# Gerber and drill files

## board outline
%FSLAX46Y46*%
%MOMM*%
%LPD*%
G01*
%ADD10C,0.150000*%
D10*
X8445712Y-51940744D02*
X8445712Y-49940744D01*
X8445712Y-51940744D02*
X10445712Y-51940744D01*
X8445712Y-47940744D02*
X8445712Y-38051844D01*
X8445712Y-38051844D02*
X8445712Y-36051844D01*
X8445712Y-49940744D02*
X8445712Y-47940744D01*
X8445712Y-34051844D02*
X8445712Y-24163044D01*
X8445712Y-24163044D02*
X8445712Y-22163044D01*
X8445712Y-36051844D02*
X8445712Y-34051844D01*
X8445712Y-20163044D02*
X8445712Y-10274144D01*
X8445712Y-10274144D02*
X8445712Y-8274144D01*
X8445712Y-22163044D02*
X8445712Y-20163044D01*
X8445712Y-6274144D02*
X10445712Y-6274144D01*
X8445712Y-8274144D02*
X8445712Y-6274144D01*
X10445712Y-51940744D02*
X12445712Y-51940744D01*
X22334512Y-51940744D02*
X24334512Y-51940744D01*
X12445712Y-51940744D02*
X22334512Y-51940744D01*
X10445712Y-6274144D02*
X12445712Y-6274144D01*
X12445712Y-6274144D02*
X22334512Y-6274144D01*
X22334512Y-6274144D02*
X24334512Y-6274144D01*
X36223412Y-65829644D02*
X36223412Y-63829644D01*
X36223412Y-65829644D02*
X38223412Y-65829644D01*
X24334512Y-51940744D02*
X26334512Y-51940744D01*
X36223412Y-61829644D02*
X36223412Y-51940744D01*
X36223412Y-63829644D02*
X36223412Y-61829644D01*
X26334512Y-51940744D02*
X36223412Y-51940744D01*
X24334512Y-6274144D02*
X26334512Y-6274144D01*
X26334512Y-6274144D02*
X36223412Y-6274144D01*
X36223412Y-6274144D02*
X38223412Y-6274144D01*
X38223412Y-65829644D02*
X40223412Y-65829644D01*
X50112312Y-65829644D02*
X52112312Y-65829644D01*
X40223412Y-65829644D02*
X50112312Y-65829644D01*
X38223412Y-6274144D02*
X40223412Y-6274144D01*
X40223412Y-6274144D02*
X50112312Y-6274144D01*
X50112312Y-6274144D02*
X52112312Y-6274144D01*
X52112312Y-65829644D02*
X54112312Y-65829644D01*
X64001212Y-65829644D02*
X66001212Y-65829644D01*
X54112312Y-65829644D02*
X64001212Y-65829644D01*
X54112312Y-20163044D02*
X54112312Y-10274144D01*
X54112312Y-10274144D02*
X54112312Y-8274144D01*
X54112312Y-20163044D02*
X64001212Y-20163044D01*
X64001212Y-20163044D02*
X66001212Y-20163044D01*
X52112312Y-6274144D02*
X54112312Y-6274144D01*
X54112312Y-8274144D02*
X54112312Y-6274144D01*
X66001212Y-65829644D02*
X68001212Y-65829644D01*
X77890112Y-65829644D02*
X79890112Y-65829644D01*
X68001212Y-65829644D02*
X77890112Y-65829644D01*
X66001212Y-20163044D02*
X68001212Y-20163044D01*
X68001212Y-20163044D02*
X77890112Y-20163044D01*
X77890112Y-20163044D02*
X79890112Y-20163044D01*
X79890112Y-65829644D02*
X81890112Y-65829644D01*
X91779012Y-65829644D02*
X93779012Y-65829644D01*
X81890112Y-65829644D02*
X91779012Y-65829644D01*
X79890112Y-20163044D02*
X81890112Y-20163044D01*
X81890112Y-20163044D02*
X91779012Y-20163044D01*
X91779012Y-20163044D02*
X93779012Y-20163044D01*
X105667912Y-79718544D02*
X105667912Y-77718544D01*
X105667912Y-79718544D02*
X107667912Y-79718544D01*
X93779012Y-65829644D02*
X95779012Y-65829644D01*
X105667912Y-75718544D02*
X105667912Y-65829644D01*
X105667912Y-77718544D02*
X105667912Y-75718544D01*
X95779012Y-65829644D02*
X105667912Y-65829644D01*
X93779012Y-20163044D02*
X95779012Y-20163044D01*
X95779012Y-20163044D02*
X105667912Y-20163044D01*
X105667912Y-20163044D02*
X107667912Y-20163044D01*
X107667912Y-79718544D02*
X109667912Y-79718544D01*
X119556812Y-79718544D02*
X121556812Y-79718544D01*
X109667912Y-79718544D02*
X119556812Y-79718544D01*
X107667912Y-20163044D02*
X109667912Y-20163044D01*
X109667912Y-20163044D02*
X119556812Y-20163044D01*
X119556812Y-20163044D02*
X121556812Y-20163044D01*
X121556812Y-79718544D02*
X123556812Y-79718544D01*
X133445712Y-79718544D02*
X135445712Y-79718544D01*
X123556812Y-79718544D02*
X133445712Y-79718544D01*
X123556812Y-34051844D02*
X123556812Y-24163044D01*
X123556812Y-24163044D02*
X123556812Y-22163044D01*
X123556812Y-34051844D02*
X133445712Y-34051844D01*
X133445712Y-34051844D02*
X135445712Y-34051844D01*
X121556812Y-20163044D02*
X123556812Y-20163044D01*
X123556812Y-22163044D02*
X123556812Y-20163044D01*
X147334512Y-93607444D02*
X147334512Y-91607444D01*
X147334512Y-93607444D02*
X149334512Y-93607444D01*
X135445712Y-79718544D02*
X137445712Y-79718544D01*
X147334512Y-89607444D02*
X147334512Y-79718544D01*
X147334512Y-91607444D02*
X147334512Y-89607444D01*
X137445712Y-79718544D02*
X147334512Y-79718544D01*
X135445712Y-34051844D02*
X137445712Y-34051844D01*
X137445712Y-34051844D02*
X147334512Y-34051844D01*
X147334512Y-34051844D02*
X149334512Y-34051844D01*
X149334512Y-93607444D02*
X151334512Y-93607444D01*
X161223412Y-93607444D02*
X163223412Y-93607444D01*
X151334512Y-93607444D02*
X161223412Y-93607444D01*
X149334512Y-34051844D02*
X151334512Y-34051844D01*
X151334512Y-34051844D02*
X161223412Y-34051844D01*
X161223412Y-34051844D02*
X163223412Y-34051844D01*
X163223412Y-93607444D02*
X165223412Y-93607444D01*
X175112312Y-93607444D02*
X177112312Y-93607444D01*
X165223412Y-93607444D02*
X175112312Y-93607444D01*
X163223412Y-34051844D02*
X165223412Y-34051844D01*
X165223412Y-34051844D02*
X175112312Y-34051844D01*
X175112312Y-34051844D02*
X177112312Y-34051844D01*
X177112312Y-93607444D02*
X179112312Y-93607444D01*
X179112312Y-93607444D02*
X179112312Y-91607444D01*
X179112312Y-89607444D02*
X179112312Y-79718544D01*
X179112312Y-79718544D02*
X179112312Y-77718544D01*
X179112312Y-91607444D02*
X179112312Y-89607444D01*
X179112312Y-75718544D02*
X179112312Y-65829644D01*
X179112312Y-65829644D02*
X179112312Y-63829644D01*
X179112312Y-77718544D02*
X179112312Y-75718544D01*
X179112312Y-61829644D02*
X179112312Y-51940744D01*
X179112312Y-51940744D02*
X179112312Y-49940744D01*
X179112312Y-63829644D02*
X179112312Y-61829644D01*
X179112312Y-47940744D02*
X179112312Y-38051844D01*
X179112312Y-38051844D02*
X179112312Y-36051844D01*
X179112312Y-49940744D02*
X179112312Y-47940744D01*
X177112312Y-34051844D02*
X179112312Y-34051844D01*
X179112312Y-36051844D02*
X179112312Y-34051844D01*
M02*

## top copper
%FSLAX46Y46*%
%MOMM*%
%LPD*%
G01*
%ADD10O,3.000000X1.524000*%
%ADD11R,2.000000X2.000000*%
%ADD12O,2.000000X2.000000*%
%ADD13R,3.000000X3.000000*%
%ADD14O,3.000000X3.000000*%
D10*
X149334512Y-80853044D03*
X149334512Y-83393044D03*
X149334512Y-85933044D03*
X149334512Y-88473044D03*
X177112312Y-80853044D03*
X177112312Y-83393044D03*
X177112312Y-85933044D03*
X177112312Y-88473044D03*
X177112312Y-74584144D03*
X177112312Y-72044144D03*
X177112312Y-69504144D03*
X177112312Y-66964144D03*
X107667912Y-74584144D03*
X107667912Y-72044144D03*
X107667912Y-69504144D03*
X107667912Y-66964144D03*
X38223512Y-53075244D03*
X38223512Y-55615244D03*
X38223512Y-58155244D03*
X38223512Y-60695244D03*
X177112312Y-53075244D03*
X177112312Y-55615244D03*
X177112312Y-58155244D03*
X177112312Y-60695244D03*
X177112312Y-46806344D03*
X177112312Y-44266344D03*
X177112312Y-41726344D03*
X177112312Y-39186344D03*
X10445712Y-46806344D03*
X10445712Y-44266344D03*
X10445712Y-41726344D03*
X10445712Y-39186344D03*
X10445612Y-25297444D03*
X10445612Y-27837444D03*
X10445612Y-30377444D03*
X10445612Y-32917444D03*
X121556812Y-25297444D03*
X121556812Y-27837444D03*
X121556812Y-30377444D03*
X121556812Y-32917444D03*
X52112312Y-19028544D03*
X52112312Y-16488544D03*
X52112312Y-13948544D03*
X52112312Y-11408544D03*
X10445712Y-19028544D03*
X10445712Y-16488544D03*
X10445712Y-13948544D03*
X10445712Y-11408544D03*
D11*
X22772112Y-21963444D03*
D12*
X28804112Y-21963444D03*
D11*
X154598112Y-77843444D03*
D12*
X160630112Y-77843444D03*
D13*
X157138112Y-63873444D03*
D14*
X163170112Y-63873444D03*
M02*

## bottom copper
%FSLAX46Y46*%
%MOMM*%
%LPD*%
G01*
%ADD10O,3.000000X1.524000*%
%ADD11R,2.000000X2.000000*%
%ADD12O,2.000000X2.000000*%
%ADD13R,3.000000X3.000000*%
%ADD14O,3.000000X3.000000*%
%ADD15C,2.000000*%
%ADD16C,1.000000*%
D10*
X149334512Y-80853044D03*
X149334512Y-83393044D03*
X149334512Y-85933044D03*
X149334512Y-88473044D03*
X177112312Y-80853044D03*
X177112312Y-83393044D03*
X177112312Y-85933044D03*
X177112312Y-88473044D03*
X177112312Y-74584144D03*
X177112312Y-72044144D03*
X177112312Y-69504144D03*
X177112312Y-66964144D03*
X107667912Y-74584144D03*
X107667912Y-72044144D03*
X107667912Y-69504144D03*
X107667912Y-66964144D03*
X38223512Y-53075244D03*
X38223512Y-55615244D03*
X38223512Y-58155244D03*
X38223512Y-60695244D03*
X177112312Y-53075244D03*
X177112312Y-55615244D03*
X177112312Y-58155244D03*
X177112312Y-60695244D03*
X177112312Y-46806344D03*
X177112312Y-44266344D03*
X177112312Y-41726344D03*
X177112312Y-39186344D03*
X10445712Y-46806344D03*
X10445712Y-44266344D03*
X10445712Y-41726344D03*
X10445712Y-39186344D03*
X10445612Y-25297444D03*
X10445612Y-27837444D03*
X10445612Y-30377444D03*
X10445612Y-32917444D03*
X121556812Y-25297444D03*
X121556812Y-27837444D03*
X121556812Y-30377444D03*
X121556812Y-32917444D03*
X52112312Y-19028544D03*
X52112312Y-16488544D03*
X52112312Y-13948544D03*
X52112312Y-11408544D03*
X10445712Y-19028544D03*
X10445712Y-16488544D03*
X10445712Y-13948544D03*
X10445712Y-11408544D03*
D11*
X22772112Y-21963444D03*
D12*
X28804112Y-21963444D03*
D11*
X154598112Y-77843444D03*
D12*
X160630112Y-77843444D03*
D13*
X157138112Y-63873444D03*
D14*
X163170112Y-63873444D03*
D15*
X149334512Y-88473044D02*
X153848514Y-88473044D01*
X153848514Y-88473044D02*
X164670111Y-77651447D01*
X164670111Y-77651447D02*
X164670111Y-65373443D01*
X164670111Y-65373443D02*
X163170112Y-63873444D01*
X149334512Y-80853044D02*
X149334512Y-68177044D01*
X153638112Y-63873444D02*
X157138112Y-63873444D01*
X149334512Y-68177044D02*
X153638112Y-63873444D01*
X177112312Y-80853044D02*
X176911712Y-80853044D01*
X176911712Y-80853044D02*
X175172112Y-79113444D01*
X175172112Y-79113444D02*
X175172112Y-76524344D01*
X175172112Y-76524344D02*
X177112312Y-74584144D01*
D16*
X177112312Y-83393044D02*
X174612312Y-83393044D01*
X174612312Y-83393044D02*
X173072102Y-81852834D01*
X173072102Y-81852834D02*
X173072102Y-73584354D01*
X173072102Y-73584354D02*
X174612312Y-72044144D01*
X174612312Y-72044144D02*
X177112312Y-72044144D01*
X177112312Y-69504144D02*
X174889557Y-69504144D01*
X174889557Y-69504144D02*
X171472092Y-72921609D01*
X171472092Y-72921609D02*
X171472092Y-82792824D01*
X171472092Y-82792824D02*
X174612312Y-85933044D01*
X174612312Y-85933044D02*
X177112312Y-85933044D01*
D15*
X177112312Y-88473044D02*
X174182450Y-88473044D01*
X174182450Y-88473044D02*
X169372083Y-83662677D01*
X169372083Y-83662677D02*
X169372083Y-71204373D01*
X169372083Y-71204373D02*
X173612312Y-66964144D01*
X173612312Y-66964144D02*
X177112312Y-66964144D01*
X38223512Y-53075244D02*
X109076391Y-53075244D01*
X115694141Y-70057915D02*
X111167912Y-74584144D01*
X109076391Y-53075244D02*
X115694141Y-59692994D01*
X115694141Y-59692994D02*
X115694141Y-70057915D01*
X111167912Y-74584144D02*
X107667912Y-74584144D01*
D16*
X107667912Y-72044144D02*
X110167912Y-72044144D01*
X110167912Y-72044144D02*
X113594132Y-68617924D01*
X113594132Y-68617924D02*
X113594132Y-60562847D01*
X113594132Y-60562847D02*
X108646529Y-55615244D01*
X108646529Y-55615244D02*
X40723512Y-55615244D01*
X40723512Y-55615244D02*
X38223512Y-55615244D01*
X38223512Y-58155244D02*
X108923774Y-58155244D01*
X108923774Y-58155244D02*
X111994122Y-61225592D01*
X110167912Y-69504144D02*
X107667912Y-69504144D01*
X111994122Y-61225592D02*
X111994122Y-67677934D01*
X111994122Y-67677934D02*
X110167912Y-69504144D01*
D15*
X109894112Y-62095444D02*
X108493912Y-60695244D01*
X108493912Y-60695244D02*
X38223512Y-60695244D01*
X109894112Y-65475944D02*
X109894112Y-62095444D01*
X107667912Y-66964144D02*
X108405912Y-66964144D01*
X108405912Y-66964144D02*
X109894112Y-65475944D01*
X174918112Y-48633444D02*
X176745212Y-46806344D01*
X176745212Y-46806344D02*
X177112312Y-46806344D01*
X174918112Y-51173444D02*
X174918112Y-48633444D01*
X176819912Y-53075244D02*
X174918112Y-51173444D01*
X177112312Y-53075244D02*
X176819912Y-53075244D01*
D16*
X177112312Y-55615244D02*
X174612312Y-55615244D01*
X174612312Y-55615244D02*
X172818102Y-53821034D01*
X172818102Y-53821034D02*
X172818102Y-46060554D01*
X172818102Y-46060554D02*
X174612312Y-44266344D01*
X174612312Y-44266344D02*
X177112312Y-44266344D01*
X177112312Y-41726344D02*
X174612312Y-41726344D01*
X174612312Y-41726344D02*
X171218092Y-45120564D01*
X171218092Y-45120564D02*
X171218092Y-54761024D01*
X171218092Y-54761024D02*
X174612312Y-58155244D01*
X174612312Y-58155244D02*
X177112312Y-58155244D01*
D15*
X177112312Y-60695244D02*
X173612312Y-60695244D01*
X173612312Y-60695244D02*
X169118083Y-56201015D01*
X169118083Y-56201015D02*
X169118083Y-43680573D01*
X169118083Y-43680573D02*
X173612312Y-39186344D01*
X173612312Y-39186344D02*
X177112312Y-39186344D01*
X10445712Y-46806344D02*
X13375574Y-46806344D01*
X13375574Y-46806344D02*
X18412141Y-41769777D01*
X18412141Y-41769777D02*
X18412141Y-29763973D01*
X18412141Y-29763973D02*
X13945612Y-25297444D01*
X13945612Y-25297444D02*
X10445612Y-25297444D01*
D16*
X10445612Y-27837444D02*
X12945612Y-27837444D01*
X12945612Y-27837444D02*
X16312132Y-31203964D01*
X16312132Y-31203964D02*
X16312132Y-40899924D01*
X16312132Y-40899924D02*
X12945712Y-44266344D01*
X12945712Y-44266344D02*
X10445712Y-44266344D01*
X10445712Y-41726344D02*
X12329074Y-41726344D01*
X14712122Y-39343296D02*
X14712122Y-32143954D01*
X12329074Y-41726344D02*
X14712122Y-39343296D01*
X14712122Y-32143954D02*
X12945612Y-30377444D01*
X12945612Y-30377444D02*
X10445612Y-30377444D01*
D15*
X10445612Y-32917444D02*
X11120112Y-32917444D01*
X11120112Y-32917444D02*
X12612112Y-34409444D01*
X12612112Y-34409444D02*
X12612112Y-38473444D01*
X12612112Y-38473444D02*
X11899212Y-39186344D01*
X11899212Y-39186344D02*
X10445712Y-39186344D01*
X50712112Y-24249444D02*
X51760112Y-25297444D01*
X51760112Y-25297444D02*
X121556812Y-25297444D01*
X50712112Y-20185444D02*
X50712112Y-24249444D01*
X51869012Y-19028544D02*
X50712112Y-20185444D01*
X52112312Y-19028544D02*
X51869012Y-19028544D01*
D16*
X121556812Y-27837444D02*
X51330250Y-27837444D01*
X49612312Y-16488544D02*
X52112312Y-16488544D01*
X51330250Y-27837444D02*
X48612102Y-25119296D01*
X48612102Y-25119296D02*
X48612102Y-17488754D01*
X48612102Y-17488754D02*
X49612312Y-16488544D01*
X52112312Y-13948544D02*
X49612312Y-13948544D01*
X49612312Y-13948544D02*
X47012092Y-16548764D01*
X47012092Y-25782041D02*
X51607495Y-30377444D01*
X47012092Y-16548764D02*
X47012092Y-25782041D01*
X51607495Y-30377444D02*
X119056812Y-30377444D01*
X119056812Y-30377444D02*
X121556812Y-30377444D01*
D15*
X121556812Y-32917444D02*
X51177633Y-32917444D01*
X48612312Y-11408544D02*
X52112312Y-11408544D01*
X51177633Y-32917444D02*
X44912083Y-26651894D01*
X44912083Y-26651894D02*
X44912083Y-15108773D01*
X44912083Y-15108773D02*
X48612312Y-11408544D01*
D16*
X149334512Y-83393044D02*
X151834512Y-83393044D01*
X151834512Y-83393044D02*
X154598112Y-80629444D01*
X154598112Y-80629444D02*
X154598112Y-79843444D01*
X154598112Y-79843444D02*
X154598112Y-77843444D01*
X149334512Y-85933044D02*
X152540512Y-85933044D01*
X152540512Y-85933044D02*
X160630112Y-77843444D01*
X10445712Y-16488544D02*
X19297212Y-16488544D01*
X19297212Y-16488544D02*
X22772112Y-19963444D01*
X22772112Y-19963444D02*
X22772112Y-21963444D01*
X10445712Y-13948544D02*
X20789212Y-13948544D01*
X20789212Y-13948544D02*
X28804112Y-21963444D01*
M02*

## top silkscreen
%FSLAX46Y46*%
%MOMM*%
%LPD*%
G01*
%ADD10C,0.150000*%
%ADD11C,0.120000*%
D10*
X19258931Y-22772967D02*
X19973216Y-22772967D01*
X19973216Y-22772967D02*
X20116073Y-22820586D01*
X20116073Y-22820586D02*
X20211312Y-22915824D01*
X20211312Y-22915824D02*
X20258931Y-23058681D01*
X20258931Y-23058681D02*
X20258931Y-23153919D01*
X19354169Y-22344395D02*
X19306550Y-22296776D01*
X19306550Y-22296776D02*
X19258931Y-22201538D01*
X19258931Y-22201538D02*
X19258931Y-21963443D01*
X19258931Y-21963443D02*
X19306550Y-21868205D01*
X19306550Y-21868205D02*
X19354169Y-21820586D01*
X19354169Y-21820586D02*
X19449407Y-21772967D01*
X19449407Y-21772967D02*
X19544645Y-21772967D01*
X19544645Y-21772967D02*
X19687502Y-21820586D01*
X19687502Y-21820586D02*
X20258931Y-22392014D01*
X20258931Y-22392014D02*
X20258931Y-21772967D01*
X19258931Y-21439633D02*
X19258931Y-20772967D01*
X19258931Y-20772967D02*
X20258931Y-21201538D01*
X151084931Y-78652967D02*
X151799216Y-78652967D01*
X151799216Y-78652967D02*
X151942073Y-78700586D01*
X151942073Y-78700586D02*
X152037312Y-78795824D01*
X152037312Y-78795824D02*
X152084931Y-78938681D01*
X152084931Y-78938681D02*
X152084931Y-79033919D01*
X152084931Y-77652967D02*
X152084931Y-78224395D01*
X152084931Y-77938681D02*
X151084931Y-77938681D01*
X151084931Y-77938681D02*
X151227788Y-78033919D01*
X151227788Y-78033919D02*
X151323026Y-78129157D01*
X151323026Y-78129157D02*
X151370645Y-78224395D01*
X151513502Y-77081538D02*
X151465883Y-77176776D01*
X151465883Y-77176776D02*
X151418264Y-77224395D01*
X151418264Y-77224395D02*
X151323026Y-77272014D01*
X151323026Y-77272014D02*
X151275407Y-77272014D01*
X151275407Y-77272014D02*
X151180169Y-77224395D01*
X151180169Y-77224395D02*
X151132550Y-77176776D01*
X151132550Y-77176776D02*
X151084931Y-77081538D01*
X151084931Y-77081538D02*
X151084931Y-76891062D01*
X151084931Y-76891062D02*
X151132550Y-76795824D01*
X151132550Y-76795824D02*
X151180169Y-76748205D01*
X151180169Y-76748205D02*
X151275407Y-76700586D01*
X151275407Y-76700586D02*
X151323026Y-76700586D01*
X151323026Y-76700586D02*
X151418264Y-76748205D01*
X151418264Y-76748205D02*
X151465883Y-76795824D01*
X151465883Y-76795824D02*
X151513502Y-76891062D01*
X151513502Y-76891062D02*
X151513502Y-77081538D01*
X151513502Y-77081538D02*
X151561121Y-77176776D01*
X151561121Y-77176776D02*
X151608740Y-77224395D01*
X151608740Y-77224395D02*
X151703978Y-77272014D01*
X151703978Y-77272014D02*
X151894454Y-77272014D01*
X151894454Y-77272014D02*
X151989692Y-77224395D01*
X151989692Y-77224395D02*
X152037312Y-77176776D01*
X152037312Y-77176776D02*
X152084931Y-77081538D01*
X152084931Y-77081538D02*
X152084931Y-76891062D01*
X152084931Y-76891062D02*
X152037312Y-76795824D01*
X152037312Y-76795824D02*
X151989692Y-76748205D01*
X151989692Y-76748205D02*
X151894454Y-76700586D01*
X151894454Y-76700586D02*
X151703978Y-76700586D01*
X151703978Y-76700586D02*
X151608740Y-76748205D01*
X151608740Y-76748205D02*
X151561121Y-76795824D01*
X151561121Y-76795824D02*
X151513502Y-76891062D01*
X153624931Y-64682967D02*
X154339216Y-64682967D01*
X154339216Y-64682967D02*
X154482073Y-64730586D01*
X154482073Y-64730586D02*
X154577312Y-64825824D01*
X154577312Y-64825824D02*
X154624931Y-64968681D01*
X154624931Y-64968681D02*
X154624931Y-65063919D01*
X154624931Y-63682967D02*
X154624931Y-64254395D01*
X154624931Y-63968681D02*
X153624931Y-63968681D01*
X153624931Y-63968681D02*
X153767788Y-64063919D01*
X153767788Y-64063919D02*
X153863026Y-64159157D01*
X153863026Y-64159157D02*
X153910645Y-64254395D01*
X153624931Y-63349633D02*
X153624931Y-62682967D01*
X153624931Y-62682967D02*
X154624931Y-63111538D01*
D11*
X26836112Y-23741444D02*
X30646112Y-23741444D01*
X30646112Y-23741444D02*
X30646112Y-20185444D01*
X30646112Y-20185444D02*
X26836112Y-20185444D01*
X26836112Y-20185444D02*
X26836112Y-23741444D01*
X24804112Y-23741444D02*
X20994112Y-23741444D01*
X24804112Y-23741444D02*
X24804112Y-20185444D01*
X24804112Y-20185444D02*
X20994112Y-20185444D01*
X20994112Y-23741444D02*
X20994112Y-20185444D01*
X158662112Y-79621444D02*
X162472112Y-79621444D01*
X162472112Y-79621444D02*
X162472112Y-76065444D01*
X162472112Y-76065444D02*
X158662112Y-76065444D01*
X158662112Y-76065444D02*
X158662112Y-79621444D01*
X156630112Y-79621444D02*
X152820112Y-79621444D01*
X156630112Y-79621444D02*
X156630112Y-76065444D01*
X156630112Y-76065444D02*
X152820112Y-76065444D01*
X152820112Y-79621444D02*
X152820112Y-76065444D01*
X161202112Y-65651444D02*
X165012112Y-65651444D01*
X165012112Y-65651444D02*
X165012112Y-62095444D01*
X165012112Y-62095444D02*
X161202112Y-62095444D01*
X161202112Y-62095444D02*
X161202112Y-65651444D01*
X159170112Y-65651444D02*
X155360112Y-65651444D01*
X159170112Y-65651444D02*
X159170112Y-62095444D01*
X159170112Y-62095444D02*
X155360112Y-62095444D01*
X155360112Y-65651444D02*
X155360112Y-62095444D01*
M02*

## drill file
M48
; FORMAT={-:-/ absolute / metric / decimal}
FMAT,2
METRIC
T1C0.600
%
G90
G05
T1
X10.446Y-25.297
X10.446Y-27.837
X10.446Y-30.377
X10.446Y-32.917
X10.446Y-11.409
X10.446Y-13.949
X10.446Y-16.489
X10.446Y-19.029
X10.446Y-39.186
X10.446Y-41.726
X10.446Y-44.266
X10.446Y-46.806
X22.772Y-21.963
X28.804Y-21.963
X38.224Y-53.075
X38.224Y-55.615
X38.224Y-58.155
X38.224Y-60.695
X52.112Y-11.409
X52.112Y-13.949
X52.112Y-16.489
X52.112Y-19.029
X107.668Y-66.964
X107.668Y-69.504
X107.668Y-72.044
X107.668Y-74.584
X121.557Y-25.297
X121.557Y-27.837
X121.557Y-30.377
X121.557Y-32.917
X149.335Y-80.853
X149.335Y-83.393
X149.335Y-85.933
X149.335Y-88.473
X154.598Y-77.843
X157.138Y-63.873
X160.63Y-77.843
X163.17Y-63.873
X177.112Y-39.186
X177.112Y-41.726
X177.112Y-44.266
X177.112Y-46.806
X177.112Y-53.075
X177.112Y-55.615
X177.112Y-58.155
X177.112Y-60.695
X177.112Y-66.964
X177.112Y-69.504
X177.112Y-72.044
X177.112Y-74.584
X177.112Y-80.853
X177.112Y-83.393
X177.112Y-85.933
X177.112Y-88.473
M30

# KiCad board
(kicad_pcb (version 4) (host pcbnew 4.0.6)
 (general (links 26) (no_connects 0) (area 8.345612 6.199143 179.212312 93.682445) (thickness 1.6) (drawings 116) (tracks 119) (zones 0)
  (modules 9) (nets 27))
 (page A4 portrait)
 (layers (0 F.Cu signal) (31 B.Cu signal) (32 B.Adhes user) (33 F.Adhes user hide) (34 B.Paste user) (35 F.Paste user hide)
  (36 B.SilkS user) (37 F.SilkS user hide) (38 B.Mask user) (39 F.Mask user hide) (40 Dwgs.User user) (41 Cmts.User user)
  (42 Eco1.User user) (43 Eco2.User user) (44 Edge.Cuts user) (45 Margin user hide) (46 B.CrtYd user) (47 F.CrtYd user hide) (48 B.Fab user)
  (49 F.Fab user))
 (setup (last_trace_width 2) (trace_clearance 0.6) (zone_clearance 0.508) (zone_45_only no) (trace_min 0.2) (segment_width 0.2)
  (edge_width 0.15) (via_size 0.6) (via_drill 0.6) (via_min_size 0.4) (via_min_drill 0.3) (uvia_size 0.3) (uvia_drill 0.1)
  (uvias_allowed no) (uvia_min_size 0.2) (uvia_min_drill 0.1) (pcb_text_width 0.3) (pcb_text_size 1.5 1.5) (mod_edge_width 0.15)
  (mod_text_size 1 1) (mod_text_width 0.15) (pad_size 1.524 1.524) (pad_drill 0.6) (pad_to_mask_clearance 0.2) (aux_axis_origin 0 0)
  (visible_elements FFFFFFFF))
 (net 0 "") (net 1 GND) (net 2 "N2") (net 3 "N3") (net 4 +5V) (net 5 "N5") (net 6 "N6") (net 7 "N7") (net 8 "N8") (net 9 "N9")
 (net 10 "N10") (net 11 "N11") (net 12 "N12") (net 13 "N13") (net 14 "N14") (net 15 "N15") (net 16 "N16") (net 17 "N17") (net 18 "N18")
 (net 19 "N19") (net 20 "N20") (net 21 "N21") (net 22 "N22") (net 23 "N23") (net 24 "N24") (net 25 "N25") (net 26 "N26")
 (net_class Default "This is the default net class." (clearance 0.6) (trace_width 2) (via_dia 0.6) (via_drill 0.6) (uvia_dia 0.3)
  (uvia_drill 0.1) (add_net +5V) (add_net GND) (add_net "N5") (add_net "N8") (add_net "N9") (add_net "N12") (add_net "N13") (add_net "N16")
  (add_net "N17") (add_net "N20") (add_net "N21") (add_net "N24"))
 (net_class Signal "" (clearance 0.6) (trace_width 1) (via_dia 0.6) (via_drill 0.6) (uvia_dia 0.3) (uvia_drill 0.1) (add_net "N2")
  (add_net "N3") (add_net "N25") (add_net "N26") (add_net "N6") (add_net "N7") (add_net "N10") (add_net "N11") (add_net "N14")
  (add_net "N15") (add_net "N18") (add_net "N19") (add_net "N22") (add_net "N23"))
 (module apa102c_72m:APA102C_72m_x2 (layer B.Cu) (at 163.223412 84.663044)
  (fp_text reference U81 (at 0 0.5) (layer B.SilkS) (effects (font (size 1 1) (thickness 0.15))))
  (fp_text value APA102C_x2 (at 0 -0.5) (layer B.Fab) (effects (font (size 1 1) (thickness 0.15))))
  (pad 1 thru_hole oval (at -13.8889 -3.81) (size 3 1.524) (drill 0.6) (layers *.Cu *.Mask) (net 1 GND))
  (pad 2 thru_hole oval (at -13.8889 -1.27) (size 3 1.524) (drill 0.6) (layers *.Cu *.Mask) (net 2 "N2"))
  (pad 3 thru_hole oval (at -13.8889 1.27) (size 3 1.524) (drill 0.6) (layers *.Cu *.Mask) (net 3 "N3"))
  (pad 4 thru_hole oval (at -13.8889 3.81) (size 3 1.524) (drill 0.6) (layers *.Cu *.Mask) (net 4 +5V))
  (pad 5 thru_hole oval (at 13.8889 -3.81) (size 3 1.524) (drill 0.6) (layers *.Cu *.Mask) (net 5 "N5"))
  (pad 6 thru_hole oval (at 13.8889 -1.27) (size 3 1.524) (drill 0.6) (layers *.Cu *.Mask) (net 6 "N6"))
  (pad 7 thru_hole oval (at 13.8889 1.27) (size 3 1.524) (drill 0.6) (layers *.Cu *.Mask) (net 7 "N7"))
  (pad 8 thru_hole oval (at 13.8889 3.81) (size 3 1.524) (drill 0.6) (layers *.Cu *.Mask) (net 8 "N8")))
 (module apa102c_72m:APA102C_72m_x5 (layer B.Cu) (at 142.390112 70.774144 180)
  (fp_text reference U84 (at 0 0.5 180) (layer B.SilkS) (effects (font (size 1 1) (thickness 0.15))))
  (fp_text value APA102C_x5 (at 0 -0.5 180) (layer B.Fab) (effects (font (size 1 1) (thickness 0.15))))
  (pad 1 thru_hole oval (at -34.7222 -3.81 180) (size 3 1.524) (drill 0.6) (layers *.Cu *.Mask) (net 5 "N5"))
  (pad 2 thru_hole oval (at -34.7222 -1.27 180) (size 3 1.524) (drill 0.6) (layers *.Cu *.Mask) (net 6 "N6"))
  (pad 3 thru_hole oval (at -34.7222 1.27 180) (size 3 1.524) (drill 0.6) (layers *.Cu *.Mask) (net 7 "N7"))
  (pad 4 thru_hole oval (at -34.7222 3.81 180) (size 3 1.524) (drill 0.6) (layers *.Cu *.Mask) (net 8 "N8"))
  (pad 5 thru_hole oval (at 34.7222 -3.81 180) (size 3 1.524) (drill 0.6) (layers *.Cu *.Mask) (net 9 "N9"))
  (pad 6 thru_hole oval (at 34.7222 -1.27 180) (size 3 1.524) (drill 0.6) (layers *.Cu *.Mask) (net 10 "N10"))
  (pad 7 thru_hole oval (at 34.7222 1.27 180) (size 3 1.524) (drill 0.6) (layers *.Cu *.Mask) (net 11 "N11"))
  (pad 8 thru_hole oval (at 34.7222 3.81 180) (size 3 1.524) (drill 0.6) (layers *.Cu *.Mask) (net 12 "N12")))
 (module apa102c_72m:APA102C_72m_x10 (layer B.Cu) (at 107.667912 56.885244)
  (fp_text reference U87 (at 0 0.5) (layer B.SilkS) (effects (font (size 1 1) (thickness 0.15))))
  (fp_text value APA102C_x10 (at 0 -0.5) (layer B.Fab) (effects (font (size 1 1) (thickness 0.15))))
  (pad 1 thru_hole oval (at -69.4444 -3.81) (size 3 1.524) (drill 0.6) (layers *.Cu *.Mask) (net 9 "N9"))
  (pad 2 thru_hole oval (at -69.4444 -1.27) (size 3 1.524) (drill 0.6) (layers *.Cu *.Mask) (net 10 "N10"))
  (pad 3 thru_hole oval (at -69.4444 1.27) (size 3 1.524) (drill 0.6) (layers *.Cu *.Mask) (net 11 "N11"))
  (pad 4 thru_hole oval (at -69.4444 3.81) (size 3 1.524) (drill 0.6) (layers *.Cu *.Mask) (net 12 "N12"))
  (pad 5 thru_hole oval (at 69.4444 -3.81) (size 3 1.524) (drill 0.6) (layers *.Cu *.Mask) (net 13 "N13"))
  (pad 6 thru_hole oval (at 69.4444 -1.27) (size 3 1.524) (drill 0.6) (layers *.Cu *.Mask) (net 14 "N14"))
  (pad 7 thru_hole oval (at 69.4444 1.27) (size 3 1.524) (drill 0.6) (layers *.Cu *.Mask) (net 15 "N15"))
  (pad 8 thru_hole oval (at 69.4444 3.81) (size 3 1.524) (drill 0.6) (layers *.Cu *.Mask) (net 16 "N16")))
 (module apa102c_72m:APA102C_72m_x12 (layer B.Cu) (at 93.779012 42.996344 180)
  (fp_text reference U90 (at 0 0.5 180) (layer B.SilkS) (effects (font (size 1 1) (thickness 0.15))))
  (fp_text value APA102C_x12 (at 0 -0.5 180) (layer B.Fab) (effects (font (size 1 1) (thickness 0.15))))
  (pad 1 thru_hole oval (at -83.3333 -3.81 180) (size 3 1.524) (drill 0.6) (layers *.Cu *.Mask) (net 13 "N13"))
  (pad 2 thru_hole oval (at -83.3333 -1.27 180) (size 3 1.524) (drill 0.6) (layers *.Cu *.Mask) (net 14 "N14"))
  (pad 3 thru_hole oval (at -83.3333 1.27 180) (size 3 1.524) (drill 0.6) (layers *.Cu *.Mask) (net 15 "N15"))
  (pad 4 thru_hole oval (at -83.3333 3.81 180) (size 3 1.524) (drill 0.6) (layers *.Cu *.Mask) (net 16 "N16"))
  (pad 5 thru_hole oval (at 83.3333 -3.81 180) (size 3 1.524) (drill 0.6) (layers *.Cu *.Mask) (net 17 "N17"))
  (pad 6 thru_hole oval (at 83.3333 -1.27 180) (size 3 1.524) (drill 0.6) (layers *.Cu *.Mask) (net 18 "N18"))
  (pad 7 thru_hole oval (at 83.3333 1.27 180) (size 3 1.524) (drill 0.6) (layers *.Cu *.Mask) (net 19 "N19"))
  (pad 8 thru_hole oval (at 83.3333 3.81 180) (size 3 1.524) (drill 0.6) (layers *.Cu *.Mask) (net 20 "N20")))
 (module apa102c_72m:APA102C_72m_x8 (layer B.Cu) (at 66.001212 29.107444)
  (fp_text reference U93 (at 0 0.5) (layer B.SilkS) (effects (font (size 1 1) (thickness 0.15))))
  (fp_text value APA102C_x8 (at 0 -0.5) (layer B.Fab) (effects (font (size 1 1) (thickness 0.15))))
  (pad 1 thru_hole oval (at -55.5556 -3.81) (size 3 1.524) (drill 0.6) (layers *.Cu *.Mask) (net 17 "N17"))
  (pad 2 thru_hole oval (at -55.5556 -1.27) (size 3 1.524) (drill 0.6) (layers *.Cu *.Mask) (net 18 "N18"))
  (pad 3 thru_hole oval (at -55.5556 1.27) (size 3 1.524) (drill 0.6) (layers *.Cu *.Mask) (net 19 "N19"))
  (pad 4 thru_hole oval (at -55.5556 3.81) (size 3 1.524) (drill 0.6) (layers *.Cu *.Mask) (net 20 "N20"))
  (pad 5 thru_hole oval (at 55.5556 -3.81) (size 3 1.524) (drill 0.6) (layers *.Cu *.Mask) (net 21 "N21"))
  (pad 6 thru_hole oval (at 55.5556 -1.27) (size 3 1.524) (drill 0.6) (layers *.Cu *.Mask) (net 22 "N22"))
  (pad 7 thru_hole oval (at 55.5556 1.27) (size 3 1.524) (drill 0.6) (layers *.Cu *.Mask) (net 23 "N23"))
  (pad 8 thru_hole oval (at 55.5556 3.81) (size 3 1.524) (drill 0.6) (layers *.Cu *.Mask) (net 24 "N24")))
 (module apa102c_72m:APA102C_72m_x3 (layer B.Cu) (at 31.279012 15.218544 180)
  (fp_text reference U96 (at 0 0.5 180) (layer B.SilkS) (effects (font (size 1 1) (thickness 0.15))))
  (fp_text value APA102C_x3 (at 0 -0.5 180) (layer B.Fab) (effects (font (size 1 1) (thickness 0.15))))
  (pad 1 thru_hole oval (at -20.8333 -3.81 180) (size 3 1.524) (drill 0.6) (layers *.Cu *.Mask) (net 21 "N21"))
  (pad 2 thru_hole oval (at -20.8333 -1.27 180) (size 3 1.524) (drill 0.6) (layers *.Cu *.Mask) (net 22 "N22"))
  (pad 3 thru_hole oval (at -20.8333 1.27 180) (size 3 1.524) (drill 0.6) (layers *.Cu *.Mask) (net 23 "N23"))
  (pad 4 thru_hole oval (at -20.8333 3.81 180) (size 3 1.524) (drill 0.6) (layers *.Cu *.Mask) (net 24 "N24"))
  (pad 5 thru_hole oval (at 20.8333 -3.81 180) (size 3 1.524) (drill 0.6) (layers *.Cu *.Mask))
  (pad 6 thru_hole oval (at 20.8333 -1.27 180) (size 3 1.524) (drill 0.6) (layers *.Cu *.Mask) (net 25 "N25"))
  (pad 7 thru_hole oval (at 20.8333 1.27 180) (size 3 1.524) (drill 0.6) (layers *.Cu *.Mask) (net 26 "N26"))
  (pad 8 thru_hole oval (at 20.8333 3.81 180) (size 3 1.524) (drill 0.6) (layers *.Cu *.Mask)))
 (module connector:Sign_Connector (layer F.Cu) (at 24.804112 21.963444 90)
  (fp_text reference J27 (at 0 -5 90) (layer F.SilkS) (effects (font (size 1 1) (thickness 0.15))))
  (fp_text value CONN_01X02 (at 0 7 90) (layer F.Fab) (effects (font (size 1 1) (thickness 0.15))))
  (fp_line (start -1.778 2.032) (end -1.778 5.842) (layer F.SilkS) (width 0.12))
  (fp_line (start -1.778 5.842) (end 1.778 5.842) (layer F.SilkS) (width 0.12))
  (fp_line (start 1.778 5.842) (end 1.778 2.032) (layer F.SilkS) (width 0.12))
  (fp_line (start 1.778 2.032) (end -1.778 2.032) (layer F.SilkS) (width 0.12))
  (fp_line (start -1.778 0) (end -1.778 -3.81) (layer F.SilkS) (width 0.12))
  (fp_line (start -1.778 0) (end 1.778 0) (layer F.SilkS) (width 0.12))
  (fp_line (start 1.778 0) (end 1.778 -3.81) (layer F.SilkS) (width 0.12))
  (fp_line (start -1.778 -3.81) (end 1.778 -3.81) (layer F.SilkS) (width 0.12))
  (pad 1 thru_hole rect (at 0 -2.032 90) (size 2 2) (drill 0.6) (layers *.Cu *.Mask) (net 25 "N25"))
  (pad 2 thru_hole oval (at 0 4 90) (size 2 2) (drill 0.6) (layers *.Cu *.Mask) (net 26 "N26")))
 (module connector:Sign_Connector (layer F.Cu) (at 156.630112 77.843444 90)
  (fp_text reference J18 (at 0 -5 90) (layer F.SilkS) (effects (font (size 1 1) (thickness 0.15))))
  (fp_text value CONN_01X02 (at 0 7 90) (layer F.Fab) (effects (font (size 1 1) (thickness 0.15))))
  (fp_line (start -1.778 2.032) (end -1.778 5.842) (layer F.SilkS) (width 0.12))
  (fp_line (start -1.778 5.842) (end 1.778 5.842) (layer F.SilkS) (width 0.12))
  (fp_line (start 1.778 5.842) (end 1.778 2.032) (layer F.SilkS) (width 0.12))
  (fp_line (start 1.778 2.032) (end -1.778 2.032) (layer F.SilkS) (width 0.12))
  (fp_line (start -1.778 0) (end -1.778 -3.81) (layer F.SilkS) (width 0.12))
  (fp_line (start -1.778 0) (end 1.778 0) (layer F.SilkS) (width 0.12))
  (fp_line (start 1.778 0) (end 1.778 -3.81) (layer F.SilkS) (width 0.12))
  (fp_line (start -1.778 -3.81) (end 1.778 -3.81) (layer F.SilkS) (width 0.12))
  (pad 1 thru_hole rect (at 0 -2.032 90) (size 2 2) (drill 0.6) (layers *.Cu *.Mask) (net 2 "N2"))
  (pad 2 thru_hole oval (at 0 4 90) (size 2 2) (drill 0.6) (layers *.Cu *.Mask) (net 3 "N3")))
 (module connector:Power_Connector (layer F.Cu) (at 159.170112 63.873444 90)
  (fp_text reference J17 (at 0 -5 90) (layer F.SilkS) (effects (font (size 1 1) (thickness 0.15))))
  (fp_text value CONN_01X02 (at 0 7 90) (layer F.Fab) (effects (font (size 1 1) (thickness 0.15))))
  (fp_line (start -1.778 2.032) (end -1.778 5.842) (layer F.SilkS) (width 0.12))
  (fp_line (start -1.778 5.842) (end 1.778 5.842) (layer F.SilkS) (width 0.12))
  (fp_line (start 1.778 5.842) (end 1.778 2.032) (layer F.SilkS) (width 0.12))
  (fp_line (start 1.778 2.032) (end -1.778 2.032) (layer F.SilkS) (width 0.12))
  (fp_line (start -1.778 0) (end -1.778 -3.81) (layer F.SilkS) (width 0.12))
  (fp_line (start -1.778 0) (end 1.778 0) (layer F.SilkS) (width 0.12))
  (fp_line (start 1.778 0) (end 1.778 -3.81) (layer F.SilkS) (width 0.12))
  (fp_line (start -1.778 -3.81) (end 1.778 -3.81) (layer F.SilkS) (width 0.12))
  (pad 1 thru_hole rect (at 0 -2.032 90) (size 3 3) (drill 0.6) (layers *.Cu *.Mask) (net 1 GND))
  (pad 2 thru_hole oval (at 0 4 90) (size 3 3) (drill 0.6) (layers *.Cu *.Mask) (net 4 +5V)))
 (gr_line (start 8.445712 51.940744) (end 8.445712 49.940744) (layer Edge.Cuts) (width 0.15))
 (gr_line (start 8.445712 51.940744) (end 10.445712 51.940744) (layer Edge.Cuts) (width 0.15))
 (gr_line (start 8.445712 47.940744) (end 8.445712 38.051844) (layer Edge.Cuts) (width 0.15))
 (gr_line (start 8.445712 38.051844) (end 8.445712 36.051844) (layer Edge.Cuts) (width 0.15))
 (gr_line (start 8.445712 49.940744) (end 8.445712 47.940744) (layer Edge.Cuts) (width 0.15))
 (gr_line (start 8.445712 34.051844) (end 8.445712 24.163044) (layer Edge.Cuts) (width 0.15))
 (gr_line (start 8.445712 24.163044) (end 8.445712 22.163044) (layer Edge.Cuts) (width 0.15))
 (gr_line (start 8.445712 36.051844) (end 8.445712 34.051844) (layer Edge.Cuts) (width 0.15))
 (gr_line (start 8.445712 20.163044) (end 8.445712 10.274144) (layer Edge.Cuts) (width 0.15))
 (gr_line (start 8.445712 10.274144) (end 8.445712 8.274144) (layer Edge.Cuts) (width 0.15))
 (gr_line (start 8.445712 22.163044) (end 8.445712 20.163044) (layer Edge.Cuts) (width 0.15))
 (gr_line (start 8.445712 6.274144) (end 10.445712 6.274144) (layer Edge.Cuts) (width 0.15))
 (gr_line (start 8.445712 8.274144) (end 8.445712 6.274144) (layer Edge.Cuts) (width 0.15))
 (gr_line (start 10.445712 51.940744) (end 12.445712 51.940744) (layer Edge.Cuts) (width 0.15))
 (gr_line (start 22.334512 51.940744) (end 24.334512 51.940744) (layer Edge.Cuts) (width 0.15))
 (gr_line (start 12.445712 51.940744) (end 22.334512 51.940744) (layer Edge.Cuts) (width 0.15))
 (gr_line (start 10.445712 6.274144) (end 12.445712 6.274144) (layer Edge.Cuts) (width 0.15))
 (gr_line (start 12.445712 6.274144) (end 22.334512 6.274144) (layer Edge.Cuts) (width 0.15))
 (gr_line (start 22.334512 6.274144) (end 24.334512 6.274144) (layer Edge.Cuts) (width 0.15))
 (gr_line (start 36.223412 65.829644) (end 36.223412 63.829644) (layer Edge.Cuts) (width 0.15))
 (gr_line (start 36.223412 65.829644) (end 38.223412 65.829644) (layer Edge.Cuts) (width 0.15))
 (gr_line (start 24.334512 51.940744) (end 26.334512 51.940744) (layer Edge.Cuts) (width 0.15))
 (gr_line (start 36.223412 61.829644) (end 36.223412 51.940744) (layer Edge.Cuts) (width 0.15))
 (gr_line (start 36.223412 63.829644) (end 36.223412 61.829644) (layer Edge.Cuts) (width 0.15))
 (gr_line (start 26.334512 51.940744) (end 36.223412 51.940744) (layer Edge.Cuts) (width 0.15))
 (gr_line (start 24.334512 6.274144) (end 26.334512 6.274144) (layer Edge.Cuts) (width 0.15))
 (gr_line (start 26.334512 6.274144) (end 36.223412 6.274144) (layer Edge.Cuts) (width 0.15))
 (gr_line (start 36.223412 6.274144) (end 38.223412 6.274144) (layer Edge.Cuts) (width 0.15))
 (gr_line (start 38.223412 65.829644) (end 40.223412 65.829644) (layer Edge.Cuts) (width 0.15))
 (gr_line (start 50.112312 65.829644) (end 52.112312 65.829644) (layer Edge.Cuts) (width 0.15))
 (gr_line (start 40.223412 65.829644) (end 50.112312 65.829644) (layer Edge.Cuts) (width 0.15))
 (gr_line (start 38.223412 6.274144) (end 40.223412 6.274144) (layer Edge.Cuts) (width 0.15))
 (gr_line (start 40.223412 6.274144) (end 50.112312 6.274144) (layer Edge.Cuts) (width 0.15))
 (gr_line (start 50.112312 6.274144) (end 52.112312 6.274144) (layer Edge.Cuts) (width 0.15))
 (gr_line (start 52.112312 65.829644) (end 54.112312 65.829644) (layer Edge.Cuts) (width 0.15))
 (gr_line (start 64.001212 65.829644) (end 66.001212 65.829644) (layer Edge.Cuts) (width 0.15))
 (gr_line (start 54.112312 65.829644) (end 64.001212 65.829644) (layer Edge.Cuts) (width 0.15))
 (gr_line (start 54.112312 20.163044) (end 54.112312 10.274144) (layer Edge.Cuts) (width 0.15))
 (gr_line (start 54.112312 10.274144) (end 54.112312 8.274144) (layer Edge.Cuts) (width 0.15))
 (gr_line (start 54.112312 20.163044) (end 64.001212 20.163044) (layer Edge.Cuts) (width 0.15))
 (gr_line (start 64.001212 20.163044) (end 66.001212 20.163044) (layer Edge.Cuts) (width 0.15))
 (gr_line (start 52.112312 6.274144) (end 54.112312 6.274144) (layer Edge.Cuts) (width 0.15))
 (gr_line (start 54.112312 8.274144) (end 54.112312 6.274144) (layer Edge.Cuts) (width 0.15))
 (gr_line (start 66.001212 65.829644) (end 68.001212 65.829644) (layer Edge.Cuts) (width 0.15))
 (gr_line (start 77.890112 65.829644) (end 79.890112 65.829644) (layer Edge.Cuts) (width 0.15))
 (gr_line (start 68.001212 65.829644) (end 77.890112 65.829644) (layer Edge.Cuts) (width 0.15))
 (gr_line (start 66.001212 20.163044) (end 68.001212 20.163044) (layer Edge.Cuts) (width 0.15))
 (gr_line (start 68.001212 20.163044) (end 77.890112 20.163044) (layer Edge.Cuts) (width 0.15))
 (gr_line (start 77.890112 20.163044) (end 79.890112 20.163044) (layer Edge.Cuts) (width 0.15))
 (gr_line (start 79.890112 65.829644) (end 81.890112 65.829644) (layer Edge.Cuts) (width 0.15))
 (gr_line (start 91.779012 65.829644) (end 93.779012 65.829644) (layer Edge.Cuts) (width 0.15))
 (gr_line (start 81.890112 65.829644) (end 91.779012 65.829644) (layer Edge.Cuts) (width 0.15))
 (gr_line (start 79.890112 20.163044) (end 81.890112 20.163044) (layer Edge.Cuts) (width 0.15))
 (gr_line (start 81.890112 20.163044) (end 91.779012 20.163044) (layer Edge.Cuts) (width 0.15))
 (gr_line (start 91.779012 20.163044) (end 93.779012 20.163044) (layer Edge.Cuts) (width 0.15))
 (gr_line (start 105.667912 79.718544) (end 105.667912 77.718544) (layer Edge.Cuts) (width 0.15))
 (gr_line (start 105.667912 79.718544) (end 107.667912 79.718544) (layer Edge.Cuts) (width 0.15))
 (gr_line (start 93.779012 65.829644) (end 95.779012 65.829644) (layer Edge.Cuts) (width 0.15))
 (gr_line (start 105.667912 75.718544) (end 105.667912 65.829644) (layer Edge.Cuts) (width 0.15))
 (gr_line (start 105.667912 77.718544) (end 105.667912 75.718544) (layer Edge.Cuts) (width 0.15))
 (gr_line (start 95.779012 65.829644) (end 105.667912 65.829644) (layer Edge.Cuts) (width 0.15))
 (gr_line (start 93.779012 20.163044) (end 95.779012 20.163044) (layer Edge.Cuts) (width 0.15))
 (gr_line (start 95.779012 20.163044) (end 105.667912 20.163044) (layer Edge.Cuts) (width 0.15))
 (gr_line (start 105.667912 20.163044) (end 107.667912 20.163044) (layer Edge.Cuts) (width 0.15))
 (gr_line (start 107.667912 79.718544) (end 109.667912 79.718544) (layer Edge.Cuts) (width 0.15))
 (gr_line (start 119.556812 79.718544) (end 121.556812 79.718544) (layer Edge.Cuts) (width 0.15))
 (gr_line (start 109.667912 79.718544) (end 119.556812 79.718544) (layer Edge.Cuts) (width 0.15))
 (gr_line (start 107.667912 20.163044) (end 109.667912 20.163044) (layer Edge.Cuts) (width 0.15))
 (gr_line (start 109.667912 20.163044) (end 119.556812 20.163044) (layer Edge.Cuts) (width 0.15))
 (gr_line (start 119.556812 20.163044) (end 121.556812 20.163044) (layer Edge.Cuts) (width 0.15))
 (gr_line (start 121.556812 79.718544) (end 123.556812 79.718544) (layer Edge.Cuts) (width 0.15))
 (gr_line (start 133.445712 79.718544) (end 135.445712 79.718544) (layer Edge.Cuts) (width 0.15))
 (gr_line (start 123.556812 79.718544) (end 133.445712 79.718544) (layer Edge.Cuts) (width 0.15))
 (gr_line (start 123.556812 34.051844) (end 123.556812 24.163044) (layer Edge.Cuts) (width 0.15))
 (gr_line (start 123.556812 24.163044) (end 123.556812 22.163044) (layer Edge.Cuts) (width 0.15))
 (gr_line (start 123.556812 34.051844) (end 133.445712 34.051844) (layer Edge.Cuts) (width 0.15))
 (gr_line (start 133.445712 34.051844) (end 135.445712 34.051844) (layer Edge.Cuts) (width 0.15))
 (gr_line (start 121.556812 20.163044) (end 123.556812 20.163044) (layer Edge.Cuts) (width 0.15))
 (gr_line (start 123.556812 22.163044) (end 123.556812 20.163044) (layer Edge.Cuts) (width 0.15))
 (gr_line (start 147.334512 93.607444) (end 147.334512 91.607444) (layer Edge.Cuts) (width 0.15))
 (gr_line (start 147.334512 93.607444) (end 149.334512 93.607444) (layer Edge.Cuts) (width 0.15))
 (gr_line (start 135.445712 79.718544) (end 137.445712 79.718544) (layer Edge.Cuts) (width 0.15))
 (gr_line (start 147.334512 89.607444) (end 147.334512 79.718544) (layer Edge.Cuts) (width 0.15))
 (gr_line (start 147.334512 91.607444) (end 147.334512 89.607444) (layer Edge.Cuts) (width 0.15))
 (gr_line (start 137.445712 79.718544) (end 147.334512 79.718544) (layer Edge.Cuts) (width 0.15))
 (gr_line (start 135.445712 34.051844) (end 137.445712 34.051844) (layer Edge.Cuts) (width 0.15))
 (gr_line (start 137.445712 34.051844) (end 147.334512 34.051844) (layer Edge.Cuts) (width 0.15))
 (gr_line (start 147.334512 34.051844) (end 149.334512 34.051844) (layer Edge.Cuts) (width 0.15))
 (gr_line (start 149.334512 93.607444) (end 151.334512 93.607444) (layer Edge.Cuts) (width 0.15))
 (gr_line (start 161.223412 93.607444) (end 163.223412 93.607444) (layer Edge.Cuts) (width 0.15))
 (gr_line (start 151.334512 93.607444) (end 161.223412 93.607444) (layer Edge.Cuts) (width 0.15))
 (gr_line (start 149.334512 34.051844) (end 151.334512 34.051844) (layer Edge.Cuts) (width 0.15))
 (gr_line (start 151.334512 34.051844) (end 161.223412 34.051844) (layer Edge.Cuts) (width 0.15))
 (gr_line (start 161.223412 34.051844) (end 163.223412 34.051844) (layer Edge.Cuts) (width 0.15))
 (gr_line (start 163.223412 93.607444) (end 165.223412 93.607444) (layer Edge.Cuts) (width 0.15))
 (gr_line (start 175.112312 93.607444) (end 177.112312 93.607444) (layer Edge.Cuts) (width 0.15))
 (gr_line (start 165.223412 93.607444) (end 175.112312 93.607444) (layer Edge.Cuts) (width 0.15))
 (gr_line (start 163.223412 34.051844) (end 165.223412 34.051844) (layer Edge.Cuts) (width 0.15))
 (gr_line (start 165.223412 34.051844) (end 175.112312 34.051844) (layer Edge.Cuts) (width 0.15))
 (gr_line (start 175.112312 34.051844) (end 177.112312 34.051844) (layer Edge.Cuts) (width 0.15))
 (gr_line (start 177.112312 93.607444) (end 179.112312 93.607444) (layer Edge.Cuts) (width 0.15))
 (gr_line (start 179.112312 93.607444) (end 179.112312 91.607444) (layer Edge.Cuts) (width 0.15))
 (gr_line (start 179.112312 89.607444) (end 179.112312 79.718544) (layer Edge.Cuts) (width 0.15))
 (gr_line (start 179.112312 79.718544) (end 179.112312 77.718544) (layer Edge.Cuts) (width 0.15))
 (gr_line (start 179.112312 91.607444) (end 179.112312 89.607444) (layer Edge.Cuts) (width 0.15))
 (gr_line (start 179.112312 75.718544) (end 179.112312 65.829644) (layer Edge.Cuts) (width 0.15))
 (gr_line (start 179.112312 65.829644) (end 179.112312 63.829644) (layer Edge.Cuts) (width 0.15))
 (gr_line (start 179.112312 77.718544) (end 179.112312 75.718544) (layer Edge.Cuts) (width 0.15))
 (gr_line (start 179.112312 61.829644) (end 179.112312 51.940744) (layer Edge.Cuts) (width 0.15))
 (gr_line (start 179.112312 51.940744) (end 179.112312 49.940744) (layer Edge.Cuts) (width 0.15))
 (gr_line (start 179.112312 63.829644) (end 179.112312 61.829644) (layer Edge.Cuts) (width 0.15))
 (gr_line (start 179.112312 47.940744) (end 179.112312 38.051844) (layer Edge.Cuts) (width 0.15))
 (gr_line (start 179.112312 38.051844) (end 179.112312 36.051844) (layer Edge.Cuts) (width 0.15))
 (gr_line (start 179.112312 49.940744) (end 179.112312 47.940744) (layer Edge.Cuts) (width 0.15))
 (gr_line (start 177.112312 34.051844) (end 179.112312 34.051844) (layer Edge.Cuts) (width 0.15))
 (gr_line (start 179.112312 36.051844) (end 179.112312 34.051844) (layer Edge.Cuts) (width 0.15))
 (segment (start 149.334512 88.473044) (end 153.848514 88.473044) (width 2) (layer B.Cu) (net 4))
 (segment (start 153.848514 88.473044) (end 164.670111 77.651447) (width 2) (layer B.Cu) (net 4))
 (segment (start 164.670111 77.651447) (end 164.670111 65.373443) (width 2) (layer B.Cu) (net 4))
 (segment (start 164.670111 65.373443) (end 163.170112 63.873444) (width 2) (layer B.Cu) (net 4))
 (segment (start 149.334512 80.853044) (end 149.334512 68.177044) (width 2) (layer B.Cu) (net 1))
 (segment (start 153.638112 63.873444) (end 157.138112 63.873444) (width 2) (layer B.Cu) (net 1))
 (segment (start 149.334512 68.177044) (end 153.638112 63.873444) (width 2) (layer B.Cu) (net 1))
 (segment (start 177.112312 80.853044) (end 176.911712 80.853044) (width 2) (layer B.Cu) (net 5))
 (segment (start 176.911712 80.853044) (end 175.172112 79.113444) (width 2) (layer B.Cu) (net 5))
 (segment (start 175.172112 79.113444) (end 175.172112 76.524344) (width 2) (layer B.Cu) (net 5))
 (segment (start 175.172112 76.524344) (end 177.112312 74.584144) (width 2) (layer B.Cu) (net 5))
 (segment (start 177.112312 83.393044) (end 174.612312 83.393044) (width 1) (layer B.Cu) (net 6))
 (segment (start 174.612312 83.393044) (end 173.072102 81.852834) (width 1) (layer B.Cu) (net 6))
 (segment (start 173.072102 81.852834) (end 173.072102 73.584354) (width 1) (layer B.Cu) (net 6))
 (segment (start 173.072102 73.584354) (end 174.612312 72.044144) (width 1) (layer B.Cu) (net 6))
 (segment (start 174.612312 72.044144) (end 177.112312 72.044144) (width 1) (layer B.Cu) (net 6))
 (segment (start 177.112312 69.504144) (end 174.889557 69.504144) (width 1) (layer B.Cu) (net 7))
 (segment (start 174.889557 69.504144) (end 171.472092 72.921609) (width 1) (layer B.Cu) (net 7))
 (segment (start 171.472092 72.921609) (end 171.472092 82.792824) (width 1) (layer B.Cu) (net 7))
 (segment (start 171.472092 82.792824) (end 174.612312 85.933044) (width 1) (layer B.Cu) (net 7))
 (segment (start 174.612312 85.933044) (end 177.112312 85.933044) (width 1) (layer B.Cu) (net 7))
 (segment (start 177.112312 88.473044) (end 174.18245 88.473044) (width 2) (layer B.Cu) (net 8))
 (segment (start 174.18245 88.473044) (end 169.372083 83.662677) (width 2) (layer B.Cu) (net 8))
 (segment (start 169.372083 83.662677) (end 169.372083 71.204373) (width 2) (layer B.Cu) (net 8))
 (segment (start 169.372083 71.204373) (end 173.612312 66.964144) (width 2) (layer B.Cu) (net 8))
 (segment (start 173.612312 66.964144) (end 177.112312 66.964144) (width 2) (layer B.Cu) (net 8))
 (segment (start 38.223512 53.075244) (end 109.076391 53.075244) (width 2) (layer B.Cu) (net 9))
 (segment (start 115.694141 70.057915) (end 111.167912 74.584144) (width 2) (layer B.Cu) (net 9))
 (segment (start 109.076391 53.075244) (end 115.694141 59.692994) (width 2) (layer B.Cu) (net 9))
 (segment (start 115.694141 59.692994) (end 115.694141 70.057915) (width 2) (layer B.Cu) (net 9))
 (segment (start 111.167912 74.584144) (end 107.667912 74.584144) (width 2) (layer B.Cu) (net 9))
 (segment (start 107.667912 72.044144) (end 110.167912 72.044144) (width 1) (layer B.Cu) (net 10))
 (segment (start 110.167912 72.044144) (end 113.594132 68.617924) (width 1) (layer B.Cu) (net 10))
 (segment (start 113.594132 68.617924) (end 113.594132 60.562847) (width 1) (layer B.Cu) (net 10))
 (segment (start 113.594132 60.562847) (end 108.646529 55.615244) (width 1) (layer B.Cu) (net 10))
 (segment (start 108.646529 55.615244) (end 40.723512 55.615244) (width 1) (layer B.Cu) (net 10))
 (segment (start 40.723512 55.615244) (end 38.223512 55.615244) (width 1) (layer B.Cu) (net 10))
 (segment (start 38.223512 58.155244) (end 108.923774 58.155244) (width 1) (layer B.Cu) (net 11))
 (segment (start 108.923774 58.155244) (end 111.994122 61.225592) (width 1) (layer B.Cu) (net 11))
 (segment (start 110.167912 69.504144) (end 107.667912 69.504144) (width 1) (layer B.Cu) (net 11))
 (segment (start 111.994122 61.225592) (end 111.994122 67.677934) (width 1) (layer B.Cu) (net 11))
 (segment (start 111.994122 67.677934) (end 110.167912 69.504144) (width 1) (layer B.Cu) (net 11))
 (segment (start 109.894112 62.095444) (end 108.493912 60.695244) (width 2) (layer B.Cu) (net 12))
 (segment (start 108.493912 60.695244) (end 38.223512 60.695244) (width 2) (layer B.Cu) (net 12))
 (segment (start 109.894112 65.475944) (end 109.894112 62.095444) (width 2) (layer B.Cu) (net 12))
 (segment (start 107.667912 66.964144) (end 108.405912 66.964144) (width 2) (layer B.Cu) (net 12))
 (segment (start 108.405912 66.964144) (end 109.894112 65.475944) (width 2) (layer B.Cu) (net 12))
 (segment (start 174.918112 48.633444) (end 176.745212 46.806344) (width 2) (layer B.Cu) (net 13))
 (segment (start 176.745212 46.806344) (end 177.112312 46.806344) (width 2) (layer B.Cu) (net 13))
 (segment (start 174.918112 51.173444) (end 174.918112 48.633444) (width 2) (layer B.Cu) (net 13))
 (segment (start 176.819912 53.075244) (end 174.918112 51.173444) (width 2) (layer B.Cu) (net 13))
 (segment (start 177.112312 53.075244) (end 176.819912 53.075244) (width 2) (layer B.Cu) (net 13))
 (segment (start 177.112312 55.615244) (end 174.612312 55.615244) (width 1) (layer B.Cu) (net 14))
 (segment (start 174.612312 55.615244) (end 172.818102 53.821034) (width 1) (layer B.Cu) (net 14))
 (segment (start 172.818102 53.821034) (end 172.818102 46.060554) (width 1) (layer B.Cu) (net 14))
 (segment (start 172.818102 46.060554) (end 174.612312 44.266344) (width 1) (layer B.Cu) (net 14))
 (segment (start 174.612312 44.266344) (end 177.112312 44.266344) (width 1) (layer B.Cu) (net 14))
 (segment (start 177.112312 41.726344) (end 174.612312 41.726344) (width 1) (layer B.Cu) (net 15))
 (segment (start 174.612312 41.726344) (end 171.218092 45.120564) (width 1) (layer B.Cu) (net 15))
 (segment (start 171.218092 45.120564) (end 171.218092 54.761024) (width 1) (layer B.Cu) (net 15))
 (segment (start 171.218092 54.761024) (end 174.612312 58.155244) (width 1) (layer B.Cu) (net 15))
 (segment (start 174.612312 58.155244) (end 177.112312 58.155244) (width 1) (layer B.Cu) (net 15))
 (segment (start 177.112312 60.695244) (end 173.612312 60.695244) (width 2) (layer B.Cu) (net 16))
 (segment (start 173.612312 60.695244) (end 169.118083 56.201015) (width 2) (layer B.Cu) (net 16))
 (segment (start 169.118083 56.201015) (end 169.118083 43.680573) (width 2) (layer B.Cu) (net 16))
 (segment (start 169.118083 43.680573) (end 173.612312 39.186344) (width 2) (layer B.Cu) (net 16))
 (segment (start 173.612312 39.186344) (end 177.112312 39.186344) (width 2) (layer B.Cu) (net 16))
 (segment (start 10.445712 46.806344) (end 13.375574 46.806344) (width 2) (layer B.Cu) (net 17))
 (segment (start 13.375574 46.806344) (end 18.412141 41.769777) (width 2) (layer B.Cu) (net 17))
 (segment (start 18.412141 41.769777) (end 18.412141 29.763973) (width 2) (layer B.Cu) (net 17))
 (segment (start 18.412141 29.763973) (end 13.945612 25.297444) (width 2) (layer B.Cu) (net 17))
 (segment (start 13.945612 25.297444) (end 10.445612 25.297444) (width 2) (layer B.Cu) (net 17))
 (segment (start 10.445612 27.837444) (end 12.945612 27.837444) (width 1) (layer B.Cu) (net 18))
 (segment (start 12.945612 27.837444) (end 16.312132 31.203964) (width 1) (layer B.Cu) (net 18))
 (segment (start 16.312132 31.203964) (end 16.312132 40.899924) (width 1) (layer B.Cu) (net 18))
 (segment (start 16.312132 40.899924) (end 12.945712 44.266344) (width 1) (layer B.Cu) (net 18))
 (segment (start 12.945712 44.266344) (end 10.445712 44.266344) (width 1) (layer B.Cu) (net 18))
 (segment (start 10.445712 41.726344) (end 12.329074 41.726344) (width 1) (layer B.Cu) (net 19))
 (segment (start 14.712122 39.343296) (end 14.712122 32.143954) (width 1) (layer B.Cu) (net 19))
 (segment (start 12.329074 41.726344) (end 14.712122 39.343296) (width 1) (layer B.Cu) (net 19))
 (segment (start 14.712122 32.143954) (end 12.945612 30.377444) (width 1) (layer B.Cu) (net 19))
 (segment (start 12.945612 30.377444) (end 10.445612 30.377444) (width 1) (layer B.Cu) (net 19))
 (segment (start 10.445612 32.917444) (end 11.120112 32.917444) (width 2) (layer B.Cu) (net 20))
 (segment (start 11.120112 32.917444) (end 12.612112 34.409444) (width 2) (layer B.Cu) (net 20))
 (segment (start 12.612112 34.409444) (end 12.612112 38.473444) (width 2) (layer B.Cu) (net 20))
 (segment (start 12.612112 38.473444) (end 11.899212 39.186344) (width 2) (layer B.Cu) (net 20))
 (segment (start 11.899212 39.186344) (end 10.445712 39.186344) (width 2) (layer B.Cu) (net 20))
 (segment (start 50.712112 24.249444) (end 51.760112 25.297444) (width 2) (layer B.Cu) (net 21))
 (segment (start 51.760112 25.297444) (end 121.556812 25.297444) (width 2) (layer B.Cu) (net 21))
 (segment (start 50.712112 20.185444) (end 50.712112 24.249444) (width 2) (layer B.Cu) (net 21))
 (segment (start 51.869012 19.028544) (end 50.712112 20.185444) (width 2) (layer B.Cu) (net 21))
 (segment (start 52.112312 19.028544) (end 51.869012 19.028544) (width 2) (layer B.Cu) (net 21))
 (segment (start 121.556812 27.837444) (end 51.33025 27.837444) (width 1) (layer B.Cu) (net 22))
 (segment (start 49.612312 16.488544) (end 52.112312 16.488544) (width 1) (layer B.Cu) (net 22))
 (segment (start 51.33025 27.837444) (end 48.612102 25.119296) (width 1) (layer B.Cu) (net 22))
 (segment (start 48.612102 25.119296) (end 48.612102 17.488754) (width 1) (layer B.Cu) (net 22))
 (segment (start 48.612102 17.488754) (end 49.612312 16.488544) (width 1) (layer B.Cu) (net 22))
 (segment (start 52.112312 13.948544) (end 49.612312 13.948544) (width 1) (layer B.Cu) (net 23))
 (segment (start 49.612312 13.948544) (end 47.012092 16.548764) (width 1) (layer B.Cu) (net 23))
 (segment (start 47.012092 25.782041) (end 51.607495 30.377444) (width 1) (layer B.Cu) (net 23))
 (segment (start 47.012092 16.548764) (end 47.012092 25.782041) (width 1) (layer B.Cu) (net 23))
 (segment (start 51.607495 30.377444) (end 119.056812 30.377444) (width 1) (layer B.Cu) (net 23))
 (segment (start 119.056812 30.377444) (end 121.556812 30.377444) (width 1) (layer B.Cu) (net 23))
 (segment (start 121.556812 32.917444) (end 51.177633 32.917444) (width 2) (layer B.Cu) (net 24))
 (segment (start 48.612312 11.408544) (end 52.112312 11.408544) (width 2) (layer B.Cu) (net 24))
 (segment (start 51.177633 32.917444) (end 44.912083 26.651894) (width 2) (layer B.Cu) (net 24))
 (segment (start 44.912083 26.651894) (end 44.912083 15.108773) (width 2) (layer B.Cu) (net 24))
 (segment (start 44.912083 15.108773) (end 48.612312 11.408544) (width 2) (layer B.Cu) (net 24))
 (segment (start 149.334512 83.393044) (end 151.834512 83.393044) (width 1) (layer B.Cu) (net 2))
 (segment (start 151.834512 83.393044) (end 154.598112 80.629444) (width 1) (layer B.Cu) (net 2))
 (segment (start 154.598112 80.629444) (end 154.598112 79.843444) (width 1) (layer B.Cu) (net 2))
 (segment (start 154.598112 79.843444) (end 154.598112 77.843444) (width 1) (layer B.Cu) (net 2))
 (segment (start 149.334512 85.933044) (end 152.540512 85.933044) (width 1) (layer B.Cu) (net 3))
 (segment (start 152.540512 85.933044) (end 160.630112 77.843444) (width 1) (layer B.Cu) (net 3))
 (segment (start 10.445712 16.488544) (end 19.297212 16.488544) (width 1) (layer B.Cu) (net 25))
 (segment (start 19.297212 16.488544) (end 22.772112 19.963444) (width 1) (layer B.Cu) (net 25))
 (segment (start 22.772112 19.963444) (end 22.772112 21.963444) (width 1) (layer B.Cu) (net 25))
 (segment (start 10.445712 13.948544) (end 20.789212 13.948544) (width 1) (layer B.Cu) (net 26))
 (segment (start 20.789212 13.948544) (end 28.804112 21.963444) (width 1) (layer B.Cu) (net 26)))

